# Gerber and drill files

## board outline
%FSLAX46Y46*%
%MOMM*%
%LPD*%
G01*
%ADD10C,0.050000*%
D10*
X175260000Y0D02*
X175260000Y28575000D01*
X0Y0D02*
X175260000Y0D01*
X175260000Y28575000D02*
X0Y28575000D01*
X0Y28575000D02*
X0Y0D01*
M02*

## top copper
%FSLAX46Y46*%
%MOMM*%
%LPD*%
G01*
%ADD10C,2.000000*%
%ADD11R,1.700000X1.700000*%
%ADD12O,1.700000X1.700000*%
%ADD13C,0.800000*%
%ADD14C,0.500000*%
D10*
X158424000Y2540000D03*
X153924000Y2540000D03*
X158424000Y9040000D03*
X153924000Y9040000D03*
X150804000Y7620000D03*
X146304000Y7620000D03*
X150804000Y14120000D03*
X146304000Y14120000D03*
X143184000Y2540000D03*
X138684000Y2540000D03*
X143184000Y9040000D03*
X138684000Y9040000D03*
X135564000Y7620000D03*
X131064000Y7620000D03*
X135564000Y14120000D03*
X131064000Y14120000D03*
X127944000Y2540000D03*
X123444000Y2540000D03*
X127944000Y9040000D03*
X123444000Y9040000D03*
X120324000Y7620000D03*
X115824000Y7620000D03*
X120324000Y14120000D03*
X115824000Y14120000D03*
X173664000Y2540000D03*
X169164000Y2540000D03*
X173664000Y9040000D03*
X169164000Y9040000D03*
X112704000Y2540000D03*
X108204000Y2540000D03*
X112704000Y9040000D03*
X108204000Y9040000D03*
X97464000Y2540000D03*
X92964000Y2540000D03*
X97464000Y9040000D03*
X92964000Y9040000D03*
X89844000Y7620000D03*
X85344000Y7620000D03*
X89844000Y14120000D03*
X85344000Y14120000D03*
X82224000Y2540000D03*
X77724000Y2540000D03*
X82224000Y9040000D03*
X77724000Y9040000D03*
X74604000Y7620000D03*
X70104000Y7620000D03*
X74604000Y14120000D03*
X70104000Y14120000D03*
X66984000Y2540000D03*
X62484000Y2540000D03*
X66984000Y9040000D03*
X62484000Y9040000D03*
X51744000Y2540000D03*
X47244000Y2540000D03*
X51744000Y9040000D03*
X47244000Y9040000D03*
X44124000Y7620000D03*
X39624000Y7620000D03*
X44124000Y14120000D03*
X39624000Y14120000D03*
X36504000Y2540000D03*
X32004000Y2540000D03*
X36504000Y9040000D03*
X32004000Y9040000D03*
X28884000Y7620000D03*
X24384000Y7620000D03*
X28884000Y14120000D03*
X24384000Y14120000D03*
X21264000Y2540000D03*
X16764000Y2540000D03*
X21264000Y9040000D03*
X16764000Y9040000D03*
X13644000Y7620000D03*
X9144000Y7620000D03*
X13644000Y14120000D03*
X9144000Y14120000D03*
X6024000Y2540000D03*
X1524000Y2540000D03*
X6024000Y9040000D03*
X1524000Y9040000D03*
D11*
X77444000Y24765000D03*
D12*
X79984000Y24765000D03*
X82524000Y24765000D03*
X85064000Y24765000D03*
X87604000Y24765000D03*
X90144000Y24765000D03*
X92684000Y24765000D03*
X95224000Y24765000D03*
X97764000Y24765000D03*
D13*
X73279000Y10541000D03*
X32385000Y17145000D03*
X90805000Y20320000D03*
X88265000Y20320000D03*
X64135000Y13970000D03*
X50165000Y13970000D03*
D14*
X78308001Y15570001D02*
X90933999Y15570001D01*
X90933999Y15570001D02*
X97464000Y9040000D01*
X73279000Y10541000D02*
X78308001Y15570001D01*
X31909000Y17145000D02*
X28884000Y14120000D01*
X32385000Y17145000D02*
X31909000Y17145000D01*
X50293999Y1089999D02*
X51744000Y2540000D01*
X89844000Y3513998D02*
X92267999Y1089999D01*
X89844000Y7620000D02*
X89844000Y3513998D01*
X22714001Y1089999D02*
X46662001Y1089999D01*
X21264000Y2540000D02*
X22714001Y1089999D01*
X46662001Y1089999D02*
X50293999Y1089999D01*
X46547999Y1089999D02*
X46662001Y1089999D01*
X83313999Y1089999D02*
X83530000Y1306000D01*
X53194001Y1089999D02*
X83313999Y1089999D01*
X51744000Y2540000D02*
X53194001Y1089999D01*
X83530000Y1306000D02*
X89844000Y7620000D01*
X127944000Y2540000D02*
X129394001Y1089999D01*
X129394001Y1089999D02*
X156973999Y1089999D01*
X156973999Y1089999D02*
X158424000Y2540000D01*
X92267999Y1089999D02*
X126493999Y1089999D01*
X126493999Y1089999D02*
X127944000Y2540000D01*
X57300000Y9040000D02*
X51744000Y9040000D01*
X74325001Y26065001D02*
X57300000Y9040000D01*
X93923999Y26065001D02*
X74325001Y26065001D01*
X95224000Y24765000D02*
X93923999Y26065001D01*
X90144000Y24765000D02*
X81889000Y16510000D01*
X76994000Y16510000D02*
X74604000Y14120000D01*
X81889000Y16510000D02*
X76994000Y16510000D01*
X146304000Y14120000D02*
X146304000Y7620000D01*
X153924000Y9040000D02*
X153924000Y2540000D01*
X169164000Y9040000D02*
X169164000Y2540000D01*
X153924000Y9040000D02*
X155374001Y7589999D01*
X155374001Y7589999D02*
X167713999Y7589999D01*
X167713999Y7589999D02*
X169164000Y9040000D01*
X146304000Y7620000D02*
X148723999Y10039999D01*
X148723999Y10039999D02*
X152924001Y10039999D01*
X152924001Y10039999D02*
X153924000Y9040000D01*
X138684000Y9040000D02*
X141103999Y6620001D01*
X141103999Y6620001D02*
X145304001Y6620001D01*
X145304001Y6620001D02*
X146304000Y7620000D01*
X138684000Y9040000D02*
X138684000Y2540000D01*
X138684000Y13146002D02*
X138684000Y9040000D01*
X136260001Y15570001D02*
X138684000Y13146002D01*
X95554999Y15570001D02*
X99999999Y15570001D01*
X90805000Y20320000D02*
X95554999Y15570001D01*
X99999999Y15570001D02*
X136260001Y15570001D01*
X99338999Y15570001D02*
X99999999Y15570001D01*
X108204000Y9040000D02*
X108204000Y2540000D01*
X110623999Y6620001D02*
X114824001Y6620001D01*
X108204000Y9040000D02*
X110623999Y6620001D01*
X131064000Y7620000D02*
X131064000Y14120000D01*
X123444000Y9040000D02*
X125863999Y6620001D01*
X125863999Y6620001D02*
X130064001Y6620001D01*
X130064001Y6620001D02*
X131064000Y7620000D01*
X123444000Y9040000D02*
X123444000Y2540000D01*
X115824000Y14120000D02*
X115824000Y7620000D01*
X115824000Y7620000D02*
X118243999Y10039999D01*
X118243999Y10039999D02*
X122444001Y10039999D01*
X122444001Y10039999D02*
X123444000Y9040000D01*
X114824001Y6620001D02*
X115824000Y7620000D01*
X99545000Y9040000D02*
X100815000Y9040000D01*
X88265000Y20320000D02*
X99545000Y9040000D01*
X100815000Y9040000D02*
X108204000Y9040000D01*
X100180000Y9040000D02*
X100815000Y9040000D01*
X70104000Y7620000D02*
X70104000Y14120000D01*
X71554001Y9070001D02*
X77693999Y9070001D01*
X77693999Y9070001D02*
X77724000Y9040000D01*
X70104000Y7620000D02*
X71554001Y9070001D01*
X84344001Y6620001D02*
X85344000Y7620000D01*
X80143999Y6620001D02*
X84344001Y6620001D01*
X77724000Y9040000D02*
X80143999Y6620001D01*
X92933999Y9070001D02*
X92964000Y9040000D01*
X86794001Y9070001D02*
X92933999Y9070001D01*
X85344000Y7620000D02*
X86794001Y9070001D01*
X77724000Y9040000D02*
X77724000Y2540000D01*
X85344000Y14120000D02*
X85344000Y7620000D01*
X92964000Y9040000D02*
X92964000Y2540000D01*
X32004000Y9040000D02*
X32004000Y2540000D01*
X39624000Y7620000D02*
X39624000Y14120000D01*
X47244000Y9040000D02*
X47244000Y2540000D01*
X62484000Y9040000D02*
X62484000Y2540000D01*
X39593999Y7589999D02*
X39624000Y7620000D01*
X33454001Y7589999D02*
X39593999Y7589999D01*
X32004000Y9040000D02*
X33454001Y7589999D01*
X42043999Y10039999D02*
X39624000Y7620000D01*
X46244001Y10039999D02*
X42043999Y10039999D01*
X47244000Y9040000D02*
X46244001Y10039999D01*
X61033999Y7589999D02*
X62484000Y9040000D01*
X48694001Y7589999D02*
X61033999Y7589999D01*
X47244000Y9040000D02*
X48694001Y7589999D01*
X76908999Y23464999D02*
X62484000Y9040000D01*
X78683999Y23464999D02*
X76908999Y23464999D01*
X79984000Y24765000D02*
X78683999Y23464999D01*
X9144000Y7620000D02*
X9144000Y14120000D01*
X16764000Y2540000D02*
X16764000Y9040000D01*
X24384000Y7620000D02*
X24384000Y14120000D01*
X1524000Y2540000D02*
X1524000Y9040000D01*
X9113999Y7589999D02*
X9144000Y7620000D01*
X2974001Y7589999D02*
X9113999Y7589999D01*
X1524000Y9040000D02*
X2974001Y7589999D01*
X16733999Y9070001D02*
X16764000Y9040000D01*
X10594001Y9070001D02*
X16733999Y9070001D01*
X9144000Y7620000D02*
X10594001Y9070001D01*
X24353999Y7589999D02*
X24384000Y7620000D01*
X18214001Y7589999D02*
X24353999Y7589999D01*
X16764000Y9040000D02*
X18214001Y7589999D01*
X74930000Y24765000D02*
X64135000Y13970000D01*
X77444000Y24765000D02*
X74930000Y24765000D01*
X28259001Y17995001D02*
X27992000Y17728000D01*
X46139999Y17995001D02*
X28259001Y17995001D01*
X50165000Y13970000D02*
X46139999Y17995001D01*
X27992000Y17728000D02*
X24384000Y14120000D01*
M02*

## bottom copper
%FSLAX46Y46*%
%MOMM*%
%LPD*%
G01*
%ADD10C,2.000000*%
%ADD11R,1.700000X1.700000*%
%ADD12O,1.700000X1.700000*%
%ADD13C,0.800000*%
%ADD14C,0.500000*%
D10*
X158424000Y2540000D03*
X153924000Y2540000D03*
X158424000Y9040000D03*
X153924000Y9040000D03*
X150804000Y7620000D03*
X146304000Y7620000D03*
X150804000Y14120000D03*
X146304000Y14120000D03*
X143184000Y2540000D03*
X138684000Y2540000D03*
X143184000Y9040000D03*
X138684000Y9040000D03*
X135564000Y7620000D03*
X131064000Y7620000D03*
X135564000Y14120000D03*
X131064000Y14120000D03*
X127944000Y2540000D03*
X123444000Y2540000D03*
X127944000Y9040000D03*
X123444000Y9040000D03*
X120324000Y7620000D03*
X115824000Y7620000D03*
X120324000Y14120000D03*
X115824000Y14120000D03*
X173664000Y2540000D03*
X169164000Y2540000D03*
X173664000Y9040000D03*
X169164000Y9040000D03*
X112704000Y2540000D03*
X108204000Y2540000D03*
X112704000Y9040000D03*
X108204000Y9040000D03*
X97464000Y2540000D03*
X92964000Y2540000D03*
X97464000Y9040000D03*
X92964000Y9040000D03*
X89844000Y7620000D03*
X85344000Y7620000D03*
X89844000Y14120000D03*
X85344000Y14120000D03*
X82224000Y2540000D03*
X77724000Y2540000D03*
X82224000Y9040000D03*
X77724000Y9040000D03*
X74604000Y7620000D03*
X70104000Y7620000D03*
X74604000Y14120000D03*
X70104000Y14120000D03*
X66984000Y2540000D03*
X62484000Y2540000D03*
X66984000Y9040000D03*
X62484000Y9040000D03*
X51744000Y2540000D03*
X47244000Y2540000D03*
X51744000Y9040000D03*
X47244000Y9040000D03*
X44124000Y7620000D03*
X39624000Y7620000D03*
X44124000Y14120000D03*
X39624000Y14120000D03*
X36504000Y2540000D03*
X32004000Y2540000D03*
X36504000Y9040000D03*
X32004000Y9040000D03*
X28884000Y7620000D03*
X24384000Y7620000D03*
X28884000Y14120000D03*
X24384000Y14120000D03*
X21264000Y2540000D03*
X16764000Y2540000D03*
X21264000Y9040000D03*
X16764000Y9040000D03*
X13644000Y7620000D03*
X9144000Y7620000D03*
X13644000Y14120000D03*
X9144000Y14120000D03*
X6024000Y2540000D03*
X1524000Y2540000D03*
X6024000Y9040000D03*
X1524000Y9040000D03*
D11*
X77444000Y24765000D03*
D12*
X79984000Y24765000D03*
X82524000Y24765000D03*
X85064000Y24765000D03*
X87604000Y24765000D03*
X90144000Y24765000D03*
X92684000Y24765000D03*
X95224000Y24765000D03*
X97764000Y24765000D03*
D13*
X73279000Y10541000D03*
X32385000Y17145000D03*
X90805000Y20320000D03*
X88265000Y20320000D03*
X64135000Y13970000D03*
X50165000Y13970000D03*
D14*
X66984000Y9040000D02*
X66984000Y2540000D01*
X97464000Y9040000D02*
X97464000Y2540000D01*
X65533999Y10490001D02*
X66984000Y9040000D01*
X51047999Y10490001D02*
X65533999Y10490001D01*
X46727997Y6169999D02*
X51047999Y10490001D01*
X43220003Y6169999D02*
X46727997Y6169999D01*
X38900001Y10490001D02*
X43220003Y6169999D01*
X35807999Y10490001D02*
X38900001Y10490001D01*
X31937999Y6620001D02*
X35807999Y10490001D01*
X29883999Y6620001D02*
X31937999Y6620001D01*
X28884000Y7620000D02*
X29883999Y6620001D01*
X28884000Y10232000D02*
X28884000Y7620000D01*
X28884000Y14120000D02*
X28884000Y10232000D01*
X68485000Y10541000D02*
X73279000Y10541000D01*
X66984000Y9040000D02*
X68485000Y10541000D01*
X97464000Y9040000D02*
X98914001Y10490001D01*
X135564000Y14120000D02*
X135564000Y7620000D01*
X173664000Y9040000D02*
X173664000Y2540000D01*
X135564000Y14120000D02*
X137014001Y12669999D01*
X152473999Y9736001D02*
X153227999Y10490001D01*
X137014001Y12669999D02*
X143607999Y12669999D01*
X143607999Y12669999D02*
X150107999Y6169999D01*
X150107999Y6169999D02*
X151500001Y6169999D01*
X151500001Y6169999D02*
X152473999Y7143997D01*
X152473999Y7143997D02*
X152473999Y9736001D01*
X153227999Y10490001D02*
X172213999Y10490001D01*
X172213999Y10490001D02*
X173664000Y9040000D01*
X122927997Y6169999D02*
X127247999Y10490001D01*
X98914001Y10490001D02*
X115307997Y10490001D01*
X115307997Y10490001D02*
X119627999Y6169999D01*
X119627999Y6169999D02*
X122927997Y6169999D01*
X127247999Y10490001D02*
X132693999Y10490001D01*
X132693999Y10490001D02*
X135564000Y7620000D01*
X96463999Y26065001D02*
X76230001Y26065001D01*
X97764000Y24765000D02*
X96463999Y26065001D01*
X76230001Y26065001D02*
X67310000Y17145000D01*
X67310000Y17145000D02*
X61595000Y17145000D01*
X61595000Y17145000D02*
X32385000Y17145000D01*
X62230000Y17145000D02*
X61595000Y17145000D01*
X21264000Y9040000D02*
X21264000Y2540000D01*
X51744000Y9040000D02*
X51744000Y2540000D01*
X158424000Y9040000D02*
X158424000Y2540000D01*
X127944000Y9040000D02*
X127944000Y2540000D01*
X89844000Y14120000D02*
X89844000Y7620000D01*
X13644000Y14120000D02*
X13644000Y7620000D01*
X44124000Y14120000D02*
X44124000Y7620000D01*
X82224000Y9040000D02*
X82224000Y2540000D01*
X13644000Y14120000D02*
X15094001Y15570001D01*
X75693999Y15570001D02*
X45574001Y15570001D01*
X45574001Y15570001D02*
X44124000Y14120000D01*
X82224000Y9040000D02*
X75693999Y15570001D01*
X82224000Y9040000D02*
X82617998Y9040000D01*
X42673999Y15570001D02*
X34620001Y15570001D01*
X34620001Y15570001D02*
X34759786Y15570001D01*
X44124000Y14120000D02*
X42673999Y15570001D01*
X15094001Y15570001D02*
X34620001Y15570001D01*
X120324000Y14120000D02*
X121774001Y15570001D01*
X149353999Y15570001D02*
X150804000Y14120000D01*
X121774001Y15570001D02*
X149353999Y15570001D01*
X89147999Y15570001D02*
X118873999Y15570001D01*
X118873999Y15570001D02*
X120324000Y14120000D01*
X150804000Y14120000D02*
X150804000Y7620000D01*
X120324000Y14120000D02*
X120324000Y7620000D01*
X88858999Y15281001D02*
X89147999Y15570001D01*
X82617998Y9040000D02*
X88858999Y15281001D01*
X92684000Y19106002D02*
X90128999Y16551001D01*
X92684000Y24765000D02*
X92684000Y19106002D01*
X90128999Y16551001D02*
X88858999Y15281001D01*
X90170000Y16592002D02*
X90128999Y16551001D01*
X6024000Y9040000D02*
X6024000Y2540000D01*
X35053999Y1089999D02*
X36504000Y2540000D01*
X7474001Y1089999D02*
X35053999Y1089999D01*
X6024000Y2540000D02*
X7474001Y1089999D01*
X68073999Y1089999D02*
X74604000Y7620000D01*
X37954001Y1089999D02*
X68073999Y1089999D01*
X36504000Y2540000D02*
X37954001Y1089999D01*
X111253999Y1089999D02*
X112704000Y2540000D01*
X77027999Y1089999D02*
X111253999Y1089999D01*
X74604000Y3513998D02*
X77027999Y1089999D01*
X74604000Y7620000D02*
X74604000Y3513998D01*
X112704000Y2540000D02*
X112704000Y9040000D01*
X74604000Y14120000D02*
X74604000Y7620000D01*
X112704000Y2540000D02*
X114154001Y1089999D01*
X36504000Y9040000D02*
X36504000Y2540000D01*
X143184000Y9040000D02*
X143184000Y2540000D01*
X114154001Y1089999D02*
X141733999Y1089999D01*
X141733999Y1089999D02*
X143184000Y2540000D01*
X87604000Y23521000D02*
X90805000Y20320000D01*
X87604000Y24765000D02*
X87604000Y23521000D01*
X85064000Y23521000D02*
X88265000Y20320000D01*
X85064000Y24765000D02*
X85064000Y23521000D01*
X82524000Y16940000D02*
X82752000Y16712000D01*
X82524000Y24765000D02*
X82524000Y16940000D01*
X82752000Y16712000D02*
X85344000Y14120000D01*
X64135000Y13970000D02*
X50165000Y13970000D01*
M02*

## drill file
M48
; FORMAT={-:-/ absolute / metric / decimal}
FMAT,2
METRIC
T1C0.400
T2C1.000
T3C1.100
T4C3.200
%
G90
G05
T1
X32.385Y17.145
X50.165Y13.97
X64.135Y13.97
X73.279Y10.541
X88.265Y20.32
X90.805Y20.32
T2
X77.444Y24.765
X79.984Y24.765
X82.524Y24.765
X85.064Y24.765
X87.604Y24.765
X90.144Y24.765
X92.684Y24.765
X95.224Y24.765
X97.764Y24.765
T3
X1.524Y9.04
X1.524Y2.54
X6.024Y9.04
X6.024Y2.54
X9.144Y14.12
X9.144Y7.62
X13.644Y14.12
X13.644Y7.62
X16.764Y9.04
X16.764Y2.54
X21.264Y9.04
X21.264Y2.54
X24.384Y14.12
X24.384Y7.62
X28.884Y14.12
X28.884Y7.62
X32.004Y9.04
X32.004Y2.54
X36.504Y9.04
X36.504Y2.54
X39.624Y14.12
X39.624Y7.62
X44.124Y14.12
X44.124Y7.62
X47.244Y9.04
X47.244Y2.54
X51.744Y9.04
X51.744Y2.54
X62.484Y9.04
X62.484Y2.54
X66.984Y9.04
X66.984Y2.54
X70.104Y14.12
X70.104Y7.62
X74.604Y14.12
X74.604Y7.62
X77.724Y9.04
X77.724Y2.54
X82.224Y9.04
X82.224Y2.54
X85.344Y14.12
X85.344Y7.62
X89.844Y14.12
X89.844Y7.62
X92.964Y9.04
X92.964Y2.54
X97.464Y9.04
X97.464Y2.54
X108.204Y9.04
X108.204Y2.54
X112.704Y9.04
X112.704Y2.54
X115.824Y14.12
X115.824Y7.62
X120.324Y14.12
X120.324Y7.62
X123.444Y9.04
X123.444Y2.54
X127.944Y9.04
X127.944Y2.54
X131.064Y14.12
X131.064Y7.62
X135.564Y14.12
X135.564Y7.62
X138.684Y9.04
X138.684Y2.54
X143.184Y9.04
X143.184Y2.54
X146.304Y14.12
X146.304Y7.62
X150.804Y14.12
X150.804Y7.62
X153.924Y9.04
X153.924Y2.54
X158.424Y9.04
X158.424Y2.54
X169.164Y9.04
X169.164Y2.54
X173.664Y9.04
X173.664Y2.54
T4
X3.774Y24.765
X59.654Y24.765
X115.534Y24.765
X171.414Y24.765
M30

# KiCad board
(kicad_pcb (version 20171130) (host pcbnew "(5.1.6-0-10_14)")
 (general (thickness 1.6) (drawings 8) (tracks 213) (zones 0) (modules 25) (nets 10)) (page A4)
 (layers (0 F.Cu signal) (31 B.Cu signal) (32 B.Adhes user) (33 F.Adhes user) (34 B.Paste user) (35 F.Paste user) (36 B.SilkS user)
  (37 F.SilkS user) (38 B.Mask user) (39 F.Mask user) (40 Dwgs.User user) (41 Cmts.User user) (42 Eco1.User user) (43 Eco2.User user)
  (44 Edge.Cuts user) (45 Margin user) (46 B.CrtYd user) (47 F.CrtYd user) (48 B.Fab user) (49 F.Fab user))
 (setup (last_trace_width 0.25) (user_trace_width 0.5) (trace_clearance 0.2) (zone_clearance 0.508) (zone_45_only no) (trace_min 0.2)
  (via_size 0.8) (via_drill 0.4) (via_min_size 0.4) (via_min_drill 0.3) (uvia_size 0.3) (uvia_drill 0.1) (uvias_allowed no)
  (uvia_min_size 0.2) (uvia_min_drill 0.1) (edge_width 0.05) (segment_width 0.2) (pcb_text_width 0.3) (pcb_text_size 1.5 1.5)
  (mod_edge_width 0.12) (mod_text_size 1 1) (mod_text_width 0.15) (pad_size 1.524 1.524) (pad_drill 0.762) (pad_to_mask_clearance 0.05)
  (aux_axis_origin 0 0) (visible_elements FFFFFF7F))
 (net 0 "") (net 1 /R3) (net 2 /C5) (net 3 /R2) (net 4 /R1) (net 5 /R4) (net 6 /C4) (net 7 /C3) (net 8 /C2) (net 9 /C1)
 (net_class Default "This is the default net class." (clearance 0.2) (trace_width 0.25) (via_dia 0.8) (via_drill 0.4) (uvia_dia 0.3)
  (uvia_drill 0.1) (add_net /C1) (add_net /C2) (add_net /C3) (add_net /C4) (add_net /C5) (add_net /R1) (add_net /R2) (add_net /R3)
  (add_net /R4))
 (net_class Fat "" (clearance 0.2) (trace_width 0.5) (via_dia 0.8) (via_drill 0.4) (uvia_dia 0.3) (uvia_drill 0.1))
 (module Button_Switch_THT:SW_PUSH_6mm (layer F.Cu) (at 153.924 -2.54 90)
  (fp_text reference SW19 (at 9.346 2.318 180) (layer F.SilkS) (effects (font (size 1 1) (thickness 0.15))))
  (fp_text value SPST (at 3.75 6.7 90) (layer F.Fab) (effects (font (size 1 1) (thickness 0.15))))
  (pad 2 thru_hole circle (at 0 4.5 180) (size 2 2) (drill 1.1) (layers *.Cu *.Mask) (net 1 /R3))
  (pad 1 thru_hole circle (at 0 0 180) (size 2 2) (drill 1.1) (layers *.Cu *.Mask) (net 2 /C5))
  (pad 2 thru_hole circle (at 6.5 4.5 180) (size 2 2) (drill 1.1) (layers *.Cu *.Mask) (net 1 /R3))
  (pad 1 thru_hole circle (at 6.5 0 180) (size 2 2) (drill 1.1) (layers *.Cu *.Mask) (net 2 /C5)))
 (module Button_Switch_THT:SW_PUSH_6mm (layer F.Cu) (at 146.304 -7.62 90)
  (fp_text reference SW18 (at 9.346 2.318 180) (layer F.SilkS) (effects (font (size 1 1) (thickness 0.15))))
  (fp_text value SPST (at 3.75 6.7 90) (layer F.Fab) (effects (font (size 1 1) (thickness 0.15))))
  (pad 2 thru_hole circle (at 0 4.5 180) (size 2 2) (drill 1.1) (layers *.Cu *.Mask) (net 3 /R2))
  (pad 1 thru_hole circle (at 0 0 180) (size 2 2) (drill 1.1) (layers *.Cu *.Mask) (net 2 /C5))
  (pad 2 thru_hole circle (at 6.5 4.5 180) (size 2 2) (drill 1.1) (layers *.Cu *.Mask) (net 3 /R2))
  (pad 1 thru_hole circle (at 6.5 0 180) (size 2 2) (drill 1.1) (layers *.Cu *.Mask) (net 2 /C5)))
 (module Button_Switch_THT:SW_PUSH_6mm (layer F.Cu) (at 138.684 -2.54 90)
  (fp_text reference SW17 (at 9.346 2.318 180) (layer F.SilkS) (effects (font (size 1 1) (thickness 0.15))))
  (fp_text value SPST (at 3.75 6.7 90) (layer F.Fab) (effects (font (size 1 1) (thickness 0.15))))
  (pad 2 thru_hole circle (at 0 4.5 180) (size 2 2) (drill 1.1) (layers *.Cu *.Mask) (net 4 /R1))
  (pad 1 thru_hole circle (at 0 0 180) (size 2 2) (drill 1.1) (layers *.Cu *.Mask) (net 2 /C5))
  (pad 2 thru_hole circle (at 6.5 4.5 180) (size 2 2) (drill 1.1) (layers *.Cu *.Mask) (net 4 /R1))
  (pad 1 thru_hole circle (at 6.5 0 180) (size 2 2) (drill 1.1) (layers *.Cu *.Mask) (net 2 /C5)))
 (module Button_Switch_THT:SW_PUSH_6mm (layer F.Cu) (at 131.064 -7.62 90)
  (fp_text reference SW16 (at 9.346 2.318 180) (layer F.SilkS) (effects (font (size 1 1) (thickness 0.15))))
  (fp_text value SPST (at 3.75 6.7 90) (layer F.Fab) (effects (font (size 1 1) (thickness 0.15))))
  (pad 2 thru_hole circle (at 0 4.5 180) (size 2 2) (drill 1.1) (layers *.Cu *.Mask) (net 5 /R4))
  (pad 1 thru_hole circle (at 0 0 180) (size 2 2) (drill 1.1) (layers *.Cu *.Mask) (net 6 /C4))
  (pad 2 thru_hole circle (at 6.5 4.5 180) (size 2 2) (drill 1.1) (layers *.Cu *.Mask) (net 5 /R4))
  (pad 1 thru_hole circle (at 6.5 0 180) (size 2 2) (drill 1.1) (layers *.Cu *.Mask) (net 6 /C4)))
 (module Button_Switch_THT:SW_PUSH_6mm (layer F.Cu) (at 123.444 -2.54 90)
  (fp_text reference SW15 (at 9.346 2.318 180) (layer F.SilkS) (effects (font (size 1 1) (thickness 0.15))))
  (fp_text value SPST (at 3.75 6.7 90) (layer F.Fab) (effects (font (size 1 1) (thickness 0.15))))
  (pad 2 thru_hole circle (at 0 4.5 180) (size 2 2) (drill 1.1) (layers *.Cu *.Mask) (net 1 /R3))
  (pad 1 thru_hole circle (at 0 0 180) (size 2 2) (drill 1.1) (layers *.Cu *.Mask) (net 6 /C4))
  (pad 2 thru_hole circle (at 6.5 4.5 180) (size 2 2) (drill 1.1) (layers *.Cu *.Mask) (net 1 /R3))
  (pad 1 thru_hole circle (at 6.5 0 180) (size 2 2) (drill 1.1) (layers *.Cu *.Mask) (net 6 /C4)))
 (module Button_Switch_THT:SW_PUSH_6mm (layer F.Cu) (at 115.824 -7.62 90)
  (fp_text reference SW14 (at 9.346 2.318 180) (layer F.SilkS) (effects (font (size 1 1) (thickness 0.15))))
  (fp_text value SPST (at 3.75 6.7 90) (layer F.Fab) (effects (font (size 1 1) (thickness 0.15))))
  (pad 2 thru_hole circle (at 0 4.5 180) (size 2 2) (drill 1.1) (layers *.Cu *.Mask) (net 3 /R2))
  (pad 1 thru_hole circle (at 0 0 180) (size 2 2) (drill 1.1) (layers *.Cu *.Mask) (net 6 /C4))
  (pad 2 thru_hole circle (at 6.5 4.5 180) (size 2 2) (drill 1.1) (layers *.Cu *.Mask) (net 3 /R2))
  (pad 1 thru_hole circle (at 6.5 0 180) (size 2 2) (drill 1.1) (layers *.Cu *.Mask) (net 6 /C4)))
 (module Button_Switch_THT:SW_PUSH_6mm (layer F.Cu) (at 169.164 -2.54 90)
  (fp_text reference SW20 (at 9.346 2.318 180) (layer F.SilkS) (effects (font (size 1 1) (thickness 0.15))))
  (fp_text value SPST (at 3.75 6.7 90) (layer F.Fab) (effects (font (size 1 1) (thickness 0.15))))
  (pad 2 thru_hole circle (at 0 4.5 180) (size 2 2) (drill 1.1) (layers *.Cu *.Mask) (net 5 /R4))
  (pad 1 thru_hole circle (at 0 0 180) (size 2 2) (drill 1.1) (layers *.Cu *.Mask) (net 2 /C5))
  (pad 2 thru_hole circle (at 6.5 4.5 180) (size 2 2) (drill 1.1) (layers *.Cu *.Mask) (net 5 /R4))
  (pad 1 thru_hole circle (at 6.5 0 180) (size 2 2) (drill 1.1) (layers *.Cu *.Mask) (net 2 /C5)))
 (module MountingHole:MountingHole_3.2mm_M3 (layer F.Cu) (at 115.534 -24.765)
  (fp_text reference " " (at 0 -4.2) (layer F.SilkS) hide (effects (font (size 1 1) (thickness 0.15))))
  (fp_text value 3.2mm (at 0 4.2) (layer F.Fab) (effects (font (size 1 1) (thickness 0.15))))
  (pad 1 np_thru_hole circle (at 0 0) (size 3.2 3.2) (drill 3.2) (layers *.Cu *.Mask)))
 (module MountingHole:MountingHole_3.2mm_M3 (layer F.Cu) (at 59.654 -24.765)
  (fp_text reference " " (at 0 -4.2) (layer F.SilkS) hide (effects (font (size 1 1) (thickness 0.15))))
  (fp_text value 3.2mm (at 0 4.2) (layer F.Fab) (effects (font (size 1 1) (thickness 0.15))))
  (pad 1 np_thru_hole circle (at 0 0) (size 3.2 3.2) (drill 3.2) (layers *.Cu *.Mask)))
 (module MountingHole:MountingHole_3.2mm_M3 (layer F.Cu) (at 171.414 -24.765)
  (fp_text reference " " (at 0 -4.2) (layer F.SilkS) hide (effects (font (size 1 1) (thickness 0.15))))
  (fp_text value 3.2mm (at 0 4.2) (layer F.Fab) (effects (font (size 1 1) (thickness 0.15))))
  (pad 1 np_thru_hole circle (at 0 0) (size 3.2 3.2) (drill 3.2) (layers *.Cu *.Mask)))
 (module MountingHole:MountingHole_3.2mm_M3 (layer F.Cu) (at 3.774 -24.765)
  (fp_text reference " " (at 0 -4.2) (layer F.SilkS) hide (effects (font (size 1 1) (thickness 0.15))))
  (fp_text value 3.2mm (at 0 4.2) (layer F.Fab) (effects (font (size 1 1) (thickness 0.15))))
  (pad 1 np_thru_hole circle (at 0 0) (size 3.2 3.2) (drill 3.2) (layers *.Cu *.Mask)))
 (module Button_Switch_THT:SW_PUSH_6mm (layer F.Cu) (at 108.204 -2.54 90)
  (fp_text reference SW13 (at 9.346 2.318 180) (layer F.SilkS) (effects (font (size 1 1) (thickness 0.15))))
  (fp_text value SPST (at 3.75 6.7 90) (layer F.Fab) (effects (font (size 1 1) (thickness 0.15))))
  (pad 2 thru_hole circle (at 0 4.5 180) (size 2 2) (drill 1.1) (layers *.Cu *.Mask) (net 4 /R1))
  (pad 1 thru_hole circle (at 0 0 180) (size 2 2) (drill 1.1) (layers *.Cu *.Mask) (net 6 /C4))
  (pad 2 thru_hole circle (at 6.5 4.5 180) (size 2 2) (drill 1.1) (layers *.Cu *.Mask) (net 4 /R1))
  (pad 1 thru_hole circle (at 6.5 0 180) (size 2 2) (drill 1.1) (layers *.Cu *.Mask) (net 6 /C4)))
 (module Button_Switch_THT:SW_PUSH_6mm (layer F.Cu) (at 92.964 -2.54 90)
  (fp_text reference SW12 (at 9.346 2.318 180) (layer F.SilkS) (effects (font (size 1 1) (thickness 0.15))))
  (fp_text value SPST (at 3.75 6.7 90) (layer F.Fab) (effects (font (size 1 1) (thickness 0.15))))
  (pad 2 thru_hole circle (at 0 4.5 180) (size 2 2) (drill 1.1) (layers *.Cu *.Mask) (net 5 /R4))
  (pad 1 thru_hole circle (at 0 0 180) (size 2 2) (drill 1.1) (layers *.Cu *.Mask) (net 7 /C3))
  (pad 2 thru_hole circle (at 6.5 4.5 180) (size 2 2) (drill 1.1) (layers *.Cu *.Mask) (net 5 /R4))
  (pad 1 thru_hole circle (at 6.5 0 180) (size 2 2) (drill 1.1) (layers *.Cu *.Mask) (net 7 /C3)))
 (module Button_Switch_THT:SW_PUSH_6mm (layer F.Cu) (at 85.344 -7.62 90)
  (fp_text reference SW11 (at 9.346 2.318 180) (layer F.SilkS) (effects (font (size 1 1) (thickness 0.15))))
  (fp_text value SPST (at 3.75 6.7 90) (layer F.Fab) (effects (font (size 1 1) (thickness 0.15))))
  (pad 2 thru_hole circle (at 0 4.5 180) (size 2 2) (drill 1.1) (layers *.Cu *.Mask) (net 1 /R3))
  (pad 1 thru_hole circle (at 0 0 180) (size 2 2) (drill 1.1) (layers *.Cu *.Mask) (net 7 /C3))
  (pad 2 thru_hole circle (at 6.5 4.5 180) (size 2 2) (drill 1.1) (layers *.Cu *.Mask) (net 1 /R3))
  (pad 1 thru_hole circle (at 6.5 0 180) (size 2 2) (drill 1.1) (layers *.Cu *.Mask) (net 7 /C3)))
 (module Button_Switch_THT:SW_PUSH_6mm (layer F.Cu) (at 77.724 -2.54 90)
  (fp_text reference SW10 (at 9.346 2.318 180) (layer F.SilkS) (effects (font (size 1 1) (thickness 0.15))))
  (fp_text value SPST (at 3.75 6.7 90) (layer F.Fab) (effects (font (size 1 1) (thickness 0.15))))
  (pad 2 thru_hole circle (at 0 4.5 180) (size 2 2) (drill 1.1) (layers *.Cu *.Mask) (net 3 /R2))
  (pad 1 thru_hole circle (at 0 0 180) (size 2 2) (drill 1.1) (layers *.Cu *.Mask) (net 7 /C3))
  (pad 2 thru_hole circle (at 6.5 4.5 180) (size 2 2) (drill 1.1) (layers *.Cu *.Mask) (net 3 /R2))
  (pad 1 thru_hole circle (at 6.5 0 180) (size 2 2) (drill 1.1) (layers *.Cu *.Mask) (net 7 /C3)))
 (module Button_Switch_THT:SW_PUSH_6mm (layer F.Cu) (at 70.104 -7.62 90)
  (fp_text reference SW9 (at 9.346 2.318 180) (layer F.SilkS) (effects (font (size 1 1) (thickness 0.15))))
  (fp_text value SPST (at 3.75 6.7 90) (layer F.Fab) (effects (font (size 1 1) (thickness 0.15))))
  (pad 2 thru_hole circle (at 0 4.5 180) (size 2 2) (drill 1.1) (layers *.Cu *.Mask) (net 4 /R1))
  (pad 1 thru_hole circle (at 0 0 180) (size 2 2) (drill 1.1) (layers *.Cu *.Mask) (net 7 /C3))
  (pad 2 thru_hole circle (at 6.5 4.5 180) (size 2 2) (drill 1.1) (layers *.Cu *.Mask) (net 4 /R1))
  (pad 1 thru_hole circle (at 6.5 0 180) (size 2 2) (drill 1.1) (layers *.Cu *.Mask) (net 7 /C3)))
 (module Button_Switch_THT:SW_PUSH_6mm (layer F.Cu) (at 62.484 -2.54 90)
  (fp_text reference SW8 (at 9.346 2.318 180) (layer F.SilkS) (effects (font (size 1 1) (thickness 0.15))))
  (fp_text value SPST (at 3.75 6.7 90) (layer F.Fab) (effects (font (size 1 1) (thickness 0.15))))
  (pad 2 thru_hole circle (at 0 4.5 180) (size 2 2) (drill 1.1) (layers *.Cu *.Mask) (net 5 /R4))
  (pad 1 thru_hole circle (at 0 0 180) (size 2 2) (drill 1.1) (layers *.Cu *.Mask) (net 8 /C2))
  (pad 2 thru_hole circle (at 6.5 4.5 180) (size 2 2) (drill 1.1) (layers *.Cu *.Mask) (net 5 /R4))
  (pad 1 thru_hole circle (at 6.5 0 180) (size 2 2) (drill 1.1) (layers *.Cu *.Mask) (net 8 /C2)))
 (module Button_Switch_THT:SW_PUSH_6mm (layer F.Cu) (at 47.244 -2.54 90)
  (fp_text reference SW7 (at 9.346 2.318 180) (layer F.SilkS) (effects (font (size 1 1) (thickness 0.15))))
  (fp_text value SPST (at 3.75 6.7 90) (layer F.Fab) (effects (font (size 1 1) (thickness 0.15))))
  (pad 2 thru_hole circle (at 0 4.5 180) (size 2 2) (drill 1.1) (layers *.Cu *.Mask) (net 1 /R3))
  (pad 1 thru_hole circle (at 0 0 180) (size 2 2) (drill 1.1) (layers *.Cu *.Mask) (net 8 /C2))
  (pad 2 thru_hole circle (at 6.5 4.5 180) (size 2 2) (drill 1.1) (layers *.Cu *.Mask) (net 1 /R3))
  (pad 1 thru_hole circle (at 6.5 0 180) (size 2 2) (drill 1.1) (layers *.Cu *.Mask) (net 8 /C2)))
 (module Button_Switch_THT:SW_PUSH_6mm (layer F.Cu) (at 39.624 -7.62 90)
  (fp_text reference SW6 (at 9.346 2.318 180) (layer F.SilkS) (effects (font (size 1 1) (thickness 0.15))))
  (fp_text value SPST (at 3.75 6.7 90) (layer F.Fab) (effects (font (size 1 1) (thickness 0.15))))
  (pad 2 thru_hole circle (at 0 4.5 180) (size 2 2) (drill 1.1) (layers *.Cu *.Mask) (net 3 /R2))
  (pad 1 thru_hole circle (at 0 0 180) (size 2 2) (drill 1.1) (layers *.Cu *.Mask) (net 8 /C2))
  (pad 2 thru_hole circle (at 6.5 4.5 180) (size 2 2) (drill 1.1) (layers *.Cu *.Mask) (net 3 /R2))
  (pad 1 thru_hole circle (at 6.5 0 180) (size 2 2) (drill 1.1) (layers *.Cu *.Mask) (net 8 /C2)))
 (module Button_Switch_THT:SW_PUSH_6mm (layer F.Cu) (at 32.004 -2.54 90)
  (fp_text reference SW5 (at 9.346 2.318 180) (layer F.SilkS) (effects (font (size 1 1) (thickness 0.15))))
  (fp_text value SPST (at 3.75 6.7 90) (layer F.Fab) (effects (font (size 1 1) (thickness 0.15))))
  (pad 2 thru_hole circle (at 0 4.5 180) (size 2 2) (drill 1.1) (layers *.Cu *.Mask) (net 4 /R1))
  (pad 1 thru_hole circle (at 0 0 180) (size 2 2) (drill 1.1) (layers *.Cu *.Mask) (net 8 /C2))
  (pad 2 thru_hole circle (at 6.5 4.5 180) (size 2 2) (drill 1.1) (layers *.Cu *.Mask) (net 4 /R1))
  (pad 1 thru_hole circle (at 6.5 0 180) (size 2 2) (drill 1.1) (layers *.Cu *.Mask) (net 8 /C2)))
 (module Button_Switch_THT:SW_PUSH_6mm (layer F.Cu) (at 24.384 -7.62 90)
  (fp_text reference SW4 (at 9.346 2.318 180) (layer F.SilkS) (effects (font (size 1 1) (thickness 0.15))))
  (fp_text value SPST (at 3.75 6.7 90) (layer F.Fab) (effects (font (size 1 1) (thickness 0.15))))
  (pad 2 thru_hole circle (at 0 4.5 180) (size 2 2) (drill 1.1) (layers *.Cu *.Mask) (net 5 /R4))
  (pad 1 thru_hole circle (at 0 0 180) (size 2 2) (drill 1.1) (layers *.Cu *.Mask) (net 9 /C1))
  (pad 2 thru_hole circle (at 6.5 4.5 180) (size 2 2) (drill 1.1) (layers *.Cu *.Mask) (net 5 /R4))
  (pad 1 thru_hole circle (at 6.5 0 180) (size 2 2) (drill 1.1) (layers *.Cu *.Mask) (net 9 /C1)))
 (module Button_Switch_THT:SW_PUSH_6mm (layer F.Cu) (at 16.764 -2.54 90)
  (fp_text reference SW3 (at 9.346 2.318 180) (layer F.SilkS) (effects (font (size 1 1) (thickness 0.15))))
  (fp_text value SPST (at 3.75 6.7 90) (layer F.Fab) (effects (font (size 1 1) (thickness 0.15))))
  (pad 2 thru_hole circle (at 0 4.5 180) (size 2 2) (drill 1.1) (layers *.Cu *.Mask) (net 1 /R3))
  (pad 1 thru_hole circle (at 0 0 180) (size 2 2) (drill 1.1) (layers *.Cu *.Mask) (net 9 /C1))
  (pad 2 thru_hole circle (at 6.5 4.5 180) (size 2 2) (drill 1.1) (layers *.Cu *.Mask) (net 1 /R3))
  (pad 1 thru_hole circle (at 6.5 0 180) (size 2 2) (drill 1.1) (layers *.Cu *.Mask) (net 9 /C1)))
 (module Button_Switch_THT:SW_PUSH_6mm (layer F.Cu) (at 9.144 -7.62 90)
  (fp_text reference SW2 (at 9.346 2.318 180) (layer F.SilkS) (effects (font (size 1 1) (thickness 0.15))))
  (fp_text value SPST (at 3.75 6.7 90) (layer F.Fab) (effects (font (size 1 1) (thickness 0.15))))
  (pad 2 thru_hole circle (at 0 4.5 180) (size 2 2) (drill 1.1) (layers *.Cu *.Mask) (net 3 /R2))
  (pad 1 thru_hole circle (at 0 0 180) (size 2 2) (drill 1.1) (layers *.Cu *.Mask) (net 9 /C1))
  (pad 2 thru_hole circle (at 6.5 4.5 180) (size 2 2) (drill 1.1) (layers *.Cu *.Mask) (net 3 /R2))
  (pad 1 thru_hole circle (at 6.5 0 180) (size 2 2) (drill 1.1) (layers *.Cu *.Mask) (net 9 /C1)))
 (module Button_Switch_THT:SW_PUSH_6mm (layer F.Cu) (at 1.524 -2.54 90)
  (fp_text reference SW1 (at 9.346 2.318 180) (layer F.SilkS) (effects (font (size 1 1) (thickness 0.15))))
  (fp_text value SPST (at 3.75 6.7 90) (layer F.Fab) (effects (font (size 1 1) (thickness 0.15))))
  (pad 2 thru_hole circle (at 0 4.5 180) (size 2 2) (drill 1.1) (layers *.Cu *.Mask) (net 4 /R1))
  (pad 1 thru_hole circle (at 0 0 180) (size 2 2) (drill 1.1) (layers *.Cu *.Mask) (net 9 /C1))
  (pad 2 thru_hole circle (at 6.5 4.5 180) (size 2 2) (drill 1.1) (layers *.Cu *.Mask) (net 4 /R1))
  (pad 1 thru_hole circle (at 6.5 0 180) (size 2 2) (drill 1.1) (layers *.Cu *.Mask) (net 9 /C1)))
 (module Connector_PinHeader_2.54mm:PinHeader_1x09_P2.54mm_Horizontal (layer F.Cu) (at 77.444 -24.765 90)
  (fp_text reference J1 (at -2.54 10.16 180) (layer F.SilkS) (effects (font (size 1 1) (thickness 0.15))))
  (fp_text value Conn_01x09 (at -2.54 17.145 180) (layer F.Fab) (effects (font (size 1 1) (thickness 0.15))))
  (pad 1 thru_hole rect (at 0 0 90) (size 1.7 1.7) (drill 1) (layers *.Cu *.Mask) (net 9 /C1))
  (pad 2 thru_hole oval (at 0 2.54 90) (size 1.7 1.7) (drill 1) (layers *.Cu *.Mask) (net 8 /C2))
  (pad 3 thru_hole oval (at 0 5.08 90) (size 1.7 1.7) (drill 1) (layers *.Cu *.Mask) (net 7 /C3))
  (pad 4 thru_hole oval (at 0 7.62 90) (size 1.7 1.7) (drill 1) (layers *.Cu *.Mask) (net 6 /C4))
  (pad 5 thru_hole oval (at 0 10.16 90) (size 1.7 1.7) (drill 1) (layers *.Cu *.Mask) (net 2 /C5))
  (pad 6 thru_hole oval (at 0 12.7 90) (size 1.7 1.7) (drill 1) (layers *.Cu *.Mask) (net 4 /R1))
  (pad 7 thru_hole oval (at 0 15.24 90) (size 1.7 1.7) (drill 1) (layers *.Cu *.Mask) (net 3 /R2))
  (pad 8 thru_hole oval (at 0 17.78 90) (size 1.7 1.7) (drill 1) (layers *.Cu *.Mask) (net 1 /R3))
  (pad 9 thru_hole oval (at 0 20.32 90) (size 1.7 1.7) (drill 1) (layers *.Cu *.Mask) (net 5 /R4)))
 (gr_line (start 175.26 0) (end 175.26 -28.575) (layer Edge.Cuts) (width 0.05))
 (gr_line (start 0 0) (end 175.26 0) (layer Edge.Cuts) (width 0.05))
 (gr_line (start 175.26 -28.575) (end 0 -28.575) (layer Edge.Cuts) (width 0.05))
 (gr_line (start 0 -28.575) (end 0 0) (layer Edge.Cuts) (width 0.05))
 (segment (start 66.984 -9.04) (end 66.984 -2.54) (width 0.5) (layer B.Cu) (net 5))
 (segment (start 97.464 -9.04) (end 97.464 -2.54) (width 0.5) (layer B.Cu) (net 5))
 (segment (start 65.533999 -10.490001) (end 66.984 -9.04) (width 0.5) (layer B.Cu) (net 5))
 (segment (start 51.047999 -10.490001) (end 65.533999 -10.490001) (width 0.5) (layer B.Cu) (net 5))
 (segment (start 46.727997 -6.169999) (end 51.047999 -10.490001) (width 0.5) (layer B.Cu) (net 5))
 (segment (start 43.220003 -6.169999) (end 46.727997 -6.169999) (width 0.5) (layer B.Cu) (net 5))
 (segment (start 38.900001 -10.490001) (end 43.220003 -6.169999) (width 0.5) (layer B.Cu) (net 5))
 (segment (start 35.807999 -10.490001) (end 38.900001 -10.490001) (width 0.5) (layer B.Cu) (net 5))
 (segment (start 31.937999 -6.620001) (end 35.807999 -10.490001) (width 0.5) (layer B.Cu) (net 5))
 (segment (start 29.883999 -6.620001) (end 31.937999 -6.620001) (width 0.5) (layer B.Cu) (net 5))
 (segment (start 28.884 -7.62) (end 29.883999 -6.620001) (width 0.5) (layer B.Cu) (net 5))
 (segment (start 28.884 -10.232) (end 28.884 -7.62) (width 0.5) (layer B.Cu) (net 5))
 (segment (start 28.884 -14.12) (end 28.884 -10.232) (width 0.5) (layer B.Cu) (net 5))
 (segment (start 68.485 -10.541) (end 73.279 -10.541) (width 0.5) (layer B.Cu) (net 5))
 (via (at 73.279 -10.541) (size 0.8) (drill 0.4) (layers F.Cu B.Cu) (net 5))
 (segment (start 66.984 -9.04) (end 68.485 -10.541) (width 0.5) (layer B.Cu) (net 5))
 (segment (start 78.308001 -15.570001) (end 90.933999 -15.570001) (width 0.5) (layer F.Cu) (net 5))
 (segment (start 90.933999 -15.570001) (end 97.464 -9.04) (width 0.5) (layer F.Cu) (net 5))
 (segment (start 73.279 -10.541) (end 78.308001 -15.570001) (width 0.5) (layer F.Cu) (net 5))
 (segment (start 97.464 -9.04) (end 98.914001 -10.490001) (width 0.5) (layer B.Cu) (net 5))
 (segment (start 135.564 -14.12) (end 135.564 -7.62) (width 0.5) (layer B.Cu) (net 5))
 (segment (start 173.664 -9.04) (end 173.664 -2.54) (width 0.5) (layer B.Cu) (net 5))
 (segment (start 135.564 -14.12) (end 137.014001 -12.669999) (width 0.5) (layer B.Cu) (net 5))
 (segment (start 152.473999 -9.736001) (end 153.227999 -10.490001) (width 0.5) (layer B.Cu) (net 5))
 (segment (start 137.014001 -12.669999) (end 143.607999 -12.669999) (width 0.5) (layer B.Cu) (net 5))
 (segment (start 143.607999 -12.669999) (end 150.107999 -6.169999) (width 0.5) (layer B.Cu) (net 5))
 (segment (start 150.107999 -6.169999) (end 151.500001 -6.169999) (width 0.5) (layer B.Cu) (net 5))
 (segment (start 151.500001 -6.169999) (end 152.473999 -7.143997) (width 0.5) (layer B.Cu) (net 5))
 (segment (start 152.473999 -7.143997) (end 152.473999 -9.736001) (width 0.5) (layer B.Cu) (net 5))
 (segment (start 153.227999 -10.490001) (end 172.213999 -10.490001) (width 0.5) (layer B.Cu) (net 5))
 (segment (start 172.213999 -10.490001) (end 173.664 -9.04) (width 0.5) (layer B.Cu) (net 5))
 (segment (start 122.927997 -6.169999) (end 127.247999 -10.490001) (width 0.5) (layer B.Cu) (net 5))
 (segment (start 98.914001 -10.490001) (end 115.307997 -10.490001) (width 0.5) (layer B.Cu) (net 5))
 (segment (start 115.307997 -10.490001) (end 119.627999 -6.169999) (width 0.5) (layer B.Cu) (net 5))
 (segment (start 119.627999 -6.169999) (end 122.927997 -6.169999) (width 0.5) (layer B.Cu) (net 5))
 (segment (start 127.247999 -10.490001) (end 132.693999 -10.490001) (width 0.5) (layer B.Cu) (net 5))
 (segment (start 132.693999 -10.490001) (end 135.564 -7.62) (width 0.5) (layer B.Cu) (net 5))
 (via (at 32.385 -17.145) (size 0.8) (drill 0.4) (layers F.Cu B.Cu) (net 5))
 (segment (start 31.909 -17.145) (end 28.884 -14.12) (width 0.5) (layer F.Cu) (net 5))
 (segment (start 32.385 -17.145) (end 31.909 -17.145) (width 0.5) (layer F.Cu) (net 5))
 (segment (start 96.463999 -26.065001) (end 76.230001 -26.065001) (width 0.5) (layer B.Cu) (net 5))
 (segment (start 97.764 -24.765) (end 96.463999 -26.065001) (width 0.5) (layer B.Cu) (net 5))
 (segment (start 76.230001 -26.065001) (end 67.31 -17.145) (width 0.5) (layer B.Cu) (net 5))
 (segment (start 67.31 -17.145) (end 61.595 -17.145) (width 0.5) (layer B.Cu) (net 5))
 (segment (start 61.595 -17.145) (end 32.385 -17.145) (width 0.5) (layer B.Cu) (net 5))
 (segment (start 62.23 -17.145) (end 61.595 -17.145) (width 0.5) (layer B.Cu) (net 5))
 (segment (start 21.264 -9.04) (end 21.264 -2.54) (width 0.5) (layer B.Cu) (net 1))
 (segment (start 51.744 -9.04) (end 51.744 -2.54) (width 0.5) (layer B.Cu) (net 1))
 (segment (start 50.293999 -1.089999) (end 51.744 -2.54) (width 0.5) (layer F.Cu) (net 1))
 (segment (start 89.844 -3.513998) (end 92.267999 -1.089999) (width 0.5) (layer F.Cu) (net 1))
 (segment (start 89.844 -7.62) (end 89.844 -3.513998) (width 0.5) (layer F.Cu) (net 1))
 (segment (start 22.714001 -1.089999) (end 46.662001 -1.089999) (width 0.5) (layer F.Cu) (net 1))
 (segment (start 21.264 -2.54) (end 22.714001 -1.089999) (width 0.5) (layer F.Cu) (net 1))
 (segment (start 46.662001 -1.089999) (end 50.293999 -1.089999) (width 0.5) (layer F.Cu) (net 1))
 (segment (start 46.547999 -1.089999) (end 46.662001 -1.089999) (width 0.5) (layer F.Cu) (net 1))
 (segment (start 83.313999 -1.089999) (end 83.53 -1.306) (width 0.5) (layer F.Cu) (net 1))
 (segment (start 53.194001 -1.089999) (end 83.313999 -1.089999) (width 0.5) (layer F.Cu) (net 1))
 (segment (start 51.744 -2.54) (end 53.194001 -1.089999) (width 0.5) (layer F.Cu) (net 1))
 (segment (start 83.53 -1.306) (end 89.844 -7.62) (width 0.5) (layer F.Cu) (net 1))
 (segment (start 127.944 -2.54) (end 129.394001 -1.089999) (width 0.5) (layer F.Cu) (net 1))
 (segment (start 129.394001 -1.089999) (end 156.973999 -1.089999) (width 0.5) (layer F.Cu) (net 1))
 (segment (start 156.973999 -1.089999) (end 158.424 -2.54) (width 0.5) (layer F.Cu) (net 1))
 (segment (start 92.267999 -1.089999) (end 126.493999 -1.089999) (width 0.5) (layer F.Cu) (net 1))
 (segment (start 126.493999 -1.089999) (end 127.944 -2.54) (width 0.5) (layer F.Cu) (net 1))
 (segment (start 158.424 -9.04) (end 158.424 -2.54) (width 0.5) (layer B.Cu) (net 1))
 (segment (start 127.944 -9.04) (end 127.944 -2.54) (width 0.5) (layer B.Cu) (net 1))
 (segment (start 89.844 -14.12) (end 89.844 -7.62) (width 0.5) (layer B.Cu) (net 1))
 (segment (start 57.3 -9.04) (end 51.744 -9.04) (width 0.5) (layer F.Cu) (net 1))
 (segment (start 74.325001 -26.065001) (end 57.3 -9.04) (width 0.5) (layer F.Cu) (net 1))
 (segment (start 93.923999 -26.065001) (end 74.325001 -26.065001) (width 0.5) (layer F.Cu) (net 1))
 (segment (start 95.224 -24.765) (end 93.923999 -26.065001) (width 0.5) (layer F.Cu) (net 1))
 (segment (start 13.644 -14.12) (end 13.644 -7.62) (width 0.5) (layer B.Cu) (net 3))
 (segment (start 44.124 -14.12) (end 44.124 -7.62) (width 0.5) (layer B.Cu) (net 3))
 (segment (start 82.224 -9.04) (end 82.224 -2.54) (width 0.5) (layer B.Cu) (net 3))
 (segment (start 13.644 -14.12) (end 15.094001 -15.570001) (width 0.5) (layer B.Cu) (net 3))
 (segment (start 75.693999 -15.570001) (end 45.574001 -15.570001) (width 0.5) (layer B.Cu) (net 3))
 (segment (start 45.574001 -15.570001) (end 44.124 -14.12) (width 0.5) (layer B.Cu) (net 3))
 (segment (start 82.224 -9.04) (end 75.693999 -15.570001) (width 0.5) (layer B.Cu) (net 3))
 (segment (start 82.224 -9.04) (end 82.617998 -9.04) (width 0.5) (layer B.Cu) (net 3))
 (segment (start 42.673999 -15.570001) (end 34.620001 -15.570001) (width 0.5) (layer B.Cu) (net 3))
 (segment (start 34.620001 -15.570001) (end 34.759786 -15.570001) (width 0.5) (layer B.Cu) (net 3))
 (segment (start 44.124 -14.12) (end 42.673999 -15.570001) (width 0.5) (layer B.Cu) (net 3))
 (segment (start 15.094001 -15.570001) (end 34.620001 -15.570001) (width 0.5) (layer B.Cu) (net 3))
 (segment (start 120.324 -14.12) (end 121.774001 -15.570001) (width 0.5) (layer B.Cu) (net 3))
 (segment (start 149.353999 -15.570001) (end 150.804 -14.12) (width 0.5) (layer B.Cu) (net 3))
 (segment (start 121.774001 -15.570001) (end 149.353999 -15.570001) (width 0.5) (layer B.Cu) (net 3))
 (segment (start 89.147999 -15.570001) (end 118.873999 -15.570001) (width 0.5) (layer B.Cu) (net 3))
 (segment (start 118.873999 -15.570001) (end 120.324 -14.12) (width 0.5) (layer B.Cu) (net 3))
 (segment (start 150.804 -14.12) (end 150.804 -7.62) (width 0.5) (layer B.Cu) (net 3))
 (segment (start 120.324 -14.12) (end 120.324 -7.62) (width 0.5) (layer B.Cu) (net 3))
 (segment (start 88.858999 -15.281001) (end 89.147999 -15.570001) (width 0.5) (layer B.Cu) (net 3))
 (segment (start 82.617998 -9.04) (end 88.858999 -15.281001) (width 0.5) (layer B.Cu) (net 3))
 (segment (start 92.684 -19.106002) (end 90.128999 -16.551001) (width 0.5) (layer B.Cu) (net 3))
 (segment (start 92.684 -24.765) (end 92.684 -19.106002) (width 0.5) (layer B.Cu) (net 3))
 (segment (start 90.128999 -16.551001) (end 88.858999 -15.281001) (width 0.5) (layer B.Cu) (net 3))
 (segment (start 90.17 -16.592002) (end 90.128999 -16.551001) (width 0.5) (layer B.Cu) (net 3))
 (segment (start 6.024 -9.04) (end 6.024 -2.54) (width 0.5) (layer B.Cu) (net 4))
 (segment (start 35.053999 -1.089999) (end 36.504 -2.54) (width 0.5) (layer B.Cu) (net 4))
 (segment (start 7.474001 -1.089999) (end 35.053999 -1.089999) (width 0.5) (layer B.Cu) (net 4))
 (segment (start 6.024 -2.54) (end 7.474001 -1.089999) (width 0.5) (layer B.Cu) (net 4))
 (segment (start 68.073999 -1.089999) (end 74.604 -7.62) (width 0.5) (layer B.Cu) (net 4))
 (segment (start 37.954001 -1.089999) (end 68.073999 -1.089999) (width 0.5) (layer B.Cu) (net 4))
 (segment (start 36.504 -2.54) (end 37.954001 -1.089999) (width 0.5) (layer B.Cu) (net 4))
 (segment (start 111.253999 -1.089999) (end 112.704 -2.54) (width 0.5) (layer B.Cu) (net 4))
 (segment (start 77.027999 -1.089999) (end 111.253999 -1.089999) (width 0.5) (layer B.Cu) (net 4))
 (segment (start 74.604 -3.513998) (end 77.027999 -1.089999) (width 0.5) (layer B.Cu) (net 4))
 (segment (start 74.604 -7.62) (end 74.604 -3.513998) (width 0.5) (layer B.Cu) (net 4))
 (segment (start 112.704 -2.54) (end 112.704 -9.04) (width 0.5) (layer B.Cu) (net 4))
 (segment (start 74.604 -14.12) (end 74.604 -7.62) (width 0.5) (layer B.Cu) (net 4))
 (segment (start 112.704 -2.54) (end 114.154001 -1.089999) (width 0.5) (layer B.Cu) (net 4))
 (segment (start 36.504 -9.04) (end 36.504 -2.54) (width 0.5) (layer B.Cu) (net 4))
 (segment (start 143.184 -9.04) (end 143.184 -2.54) (width 0.5) (layer B.Cu) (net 4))
 (segment (start 114.154001 -1.089999) (end 141.733999 -1.089999) (width 0.5) (layer B.Cu) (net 4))
 (segment (start 141.733999 -1.089999) (end 143.184 -2.54) (width 0.5) (layer B.Cu) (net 4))
 (segment (start 90.144 -24.765) (end 81.889 -16.51) (width 0.5) (layer F.Cu) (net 4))
 (segment (start 76.994 -16.51) (end 74.604 -14.12) (width 0.5) (layer F.Cu) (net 4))
 (segment (start 81.889 -16.51) (end 76.994 -16.51) (width 0.5) (layer F.Cu) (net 4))
 (segment (start 146.304 -14.12) (end 146.304 -7.62) (width 0.5) (layer F.Cu) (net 2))
 (segment (start 153.924 -9.04) (end 153.924 -2.54) (width 0.5) (layer F.Cu) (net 2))
 (segment (start 169.164 -9.04) (end 169.164 -2.54) (width 0.5) (layer F.Cu) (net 2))
 (segment (start 153.924 -9.04) (end 155.374001 -7.589999) (width 0.5) (layer F.Cu) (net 2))
 (segment (start 155.374001 -7.589999) (end 167.713999 -7.589999) (width 0.5) (layer F.Cu) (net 2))
 (segment (start 167.713999 -7.589999) (end 169.164 -9.04) (width 0.5) (layer F.Cu) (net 2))
 (segment (start 146.304 -7.62) (end 148.723999 -10.039999) (width 0.5) (layer F.Cu) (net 2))
 (segment (start 148.723999 -10.039999) (end 152.924001 -10.039999) (width 0.5) (layer F.Cu) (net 2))
 (segment (start 152.924001 -10.039999) (end 153.924 -9.04) (width 0.5) (layer F.Cu) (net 2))
 (segment (start 138.684 -9.04) (end 141.103999 -6.620001) (width 0.5) (layer F.Cu) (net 2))
 (segment (start 141.103999 -6.620001) (end 145.304001 -6.620001) (width 0.5) (layer F.Cu) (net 2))
 (segment (start 145.304001 -6.620001) (end 146.304 -7.62) (width 0.5) (layer F.Cu) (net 2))
 (segment (start 138.684 -9.04) (end 138.684 -2.54) (width 0.5) (layer F.Cu) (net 2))
 (segment (start 138.684 -13.146002) (end 138.684 -9.04) (width 0.5) (layer F.Cu) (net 2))
 (segment (start 136.260001 -15.570001) (end 138.684 -13.146002) (width 0.5) (layer F.Cu) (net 2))
 (segment (start 87.604 -23.521) (end 90.805 -20.32) (width 0.5) (layer B.Cu) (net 2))
 (via (at 90.805 -20.32) (size 0.8) (drill 0.4) (layers F.Cu B.Cu) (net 2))
 (segment (start 87.604 -24.765) (end 87.604 -23.521) (width 0.5) (layer B.Cu) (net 2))
 (segment (start 95.554999 -15.570001) (end 99.999999 -15.570001) (width 0.5) (layer F.Cu) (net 2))
 (segment (start 90.805 -20.32) (end 95.554999 -15.570001) (width 0.5) (layer F.Cu) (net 2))
 (segment (start 99.999999 -15.570001) (end 136.260001 -15.570001) (width 0.5) (layer F.Cu) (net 2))
 (segment (start 99.338999 -15.570001) (end 99.999999 -15.570001) (width 0.5) (layer F.Cu) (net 2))
 (segment (start 108.204 -9.04) (end 108.204 -2.54) (width 0.5) (layer F.Cu) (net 6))
 (segment (start 110.623999 -6.620001) (end 114.824001 -6.620001) (width 0.5) (layer F.Cu) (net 6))
 (segment (start 108.204 -9.04) (end 110.623999 -6.620001) (width 0.5) (layer F.Cu) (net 6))
 (segment (start 131.064 -7.62) (end 131.064 -14.12) (width 0.5) (layer F.Cu) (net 6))
 (segment (start 123.444 -9.04) (end 125.863999 -6.620001) (width 0.5) (layer F.Cu) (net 6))
 (segment (start 125.863999 -6.620001) (end 130.064001 -6.620001) (width 0.5) (layer F.Cu) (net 6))
 (segment (start 130.064001 -6.620001) (end 131.064 -7.62) (width 0.5) (layer F.Cu) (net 6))
 (segment (start 123.444 -9.04) (end 123.444 -2.54) (width 0.5) (layer F.Cu) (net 6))
 (segment (start 115.824 -14.12) (end 115.824 -7.62) (width 0.5) (layer F.Cu) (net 6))
 (segment (start 115.824 -7.62) (end 118.243999 -10.039999) (width 0.5) (layer F.Cu) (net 6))
 (segment (start 118.243999 -10.039999) (end 122.444001 -10.039999) (width 0.5) (layer F.Cu) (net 6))
 (segment (start 122.444001 -10.039999) (end 123.444 -9.04) (width 0.5) (layer F.Cu) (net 6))
 (segment (start 114.824001 -6.620001) (end 115.824 -7.62) (width 0.5) (layer F.Cu) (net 6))
 (via (at 88.265 -20.32) (size 0.8) (drill 0.4) (layers F.Cu B.Cu) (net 6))
 (segment (start 85.064 -23.521) (end 88.265 -20.32) (width 0.5) (layer B.Cu) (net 6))
 (segment (start 85.064 -24.765) (end 85.064 -23.521) (width 0.5) (layer B.Cu) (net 6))
 (segment (start 99.545 -9.04) (end 100.815 -9.04) (width 0.5) (layer F.Cu) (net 6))
 (segment (start 88.265 -20.32) (end 99.545 -9.04) (width 0.5) (layer F.Cu) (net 6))
 (segment (start 100.815 -9.04) (end 108.204 -9.04) (width 0.5) (layer F.Cu) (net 6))
 (segment (start 100.18 -9.04) (end 100.815 -9.04) (width 0.5) (layer F.Cu) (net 6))
 (segment (start 70.104 -7.62) (end 70.104 -14.12) (width 0.5) (layer F.Cu) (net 7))
 (segment (start 71.554001 -9.070001) (end 77.693999 -9.070001) (width 0.5) (layer F.Cu) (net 7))
 (segment (start 77.693999 -9.070001) (end 77.724 -9.04) (width 0.5) (layer F.Cu) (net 7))
 (segment (start 70.104 -7.62) (end 71.554001 -9.070001) (width 0.5) (layer F.Cu) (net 7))
 (segment (start 84.344001 -6.620001) (end 85.344 -7.62) (width 0.5) (layer F.Cu) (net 7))
 (segment (start 80.143999 -6.620001) (end 84.344001 -6.620001) (width 0.5) (layer F.Cu) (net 7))
 (segment (start 77.724 -9.04) (end 80.143999 -6.620001) (width 0.5) (layer F.Cu) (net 7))
 (segment (start 92.933999 -9.070001) (end 92.964 -9.04) (width 0.5) (layer F.Cu) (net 7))
 (segment (start 86.794001 -9.070001) (end 92.933999 -9.070001) (width 0.5) (layer F.Cu) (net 7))
 (segment (start 85.344 -7.62) (end 86.794001 -9.070001) (width 0.5) (layer F.Cu) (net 7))
 (segment (start 77.724 -9.04) (end 77.724 -2.54) (width 0.5) (layer F.Cu) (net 7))
 (segment (start 85.344 -14.12) (end 85.344 -7.62) (width 0.5) (layer F.Cu) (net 7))
 (segment (start 92.964 -9.04) (end 92.964 -2.54) (width 0.5) (layer F.Cu) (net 7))
 (segment (start 82.524 -16.94) (end 82.752 -16.712) (width 0.5) (layer B.Cu) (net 7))
 (segment (start 82.524 -24.765) (end 82.524 -16.94) (width 0.5) (layer B.Cu) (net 7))
 (segment (start 82.752 -16.712) (end 85.344 -14.12) (width 0.5) (layer B.Cu) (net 7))
 (segment (start 32.004 -9.04) (end 32.004 -2.54) (width 0.5) (layer F.Cu) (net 8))
 (segment (start 39.624 -7.62) (end 39.624 -14.12) (width 0.5) (layer F.Cu) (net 8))
 (segment (start 47.244 -9.04) (end 47.244 -2.54) (width 0.5) (layer F.Cu) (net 8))
 (segment (start 62.484 -9.04) (end 62.484 -2.54) (width 0.5) (layer F.Cu) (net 8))
 (segment (start 39.593999 -7.589999) (end 39.624 -7.62) (width 0.5) (layer F.Cu) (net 8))
 (segment (start 33.454001 -7.589999) (end 39.593999 -7.589999) (width 0.5) (layer F.Cu) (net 8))
 (segment (start 32.004 -9.04) (end 33.454001 -7.589999) (width 0.5) (layer F.Cu) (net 8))
 (segment (start 42.043999 -10.039999) (end 39.624 -7.62) (width 0.5) (layer F.Cu) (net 8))
 (segment (start 46.244001 -10.039999) (end 42.043999 -10.039999) (width 0.5) (layer F.Cu) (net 8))
 (segment (start 47.244 -9.04) (end 46.244001 -10.039999) (width 0.5) (layer F.Cu) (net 8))
 (segment (start 61.033999 -7.589999) (end 62.484 -9.04) (width 0.5) (layer F.Cu) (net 8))
 (segment (start 48.694001 -7.589999) (end 61.033999 -7.589999) (width 0.5) (layer F.Cu) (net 8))
 (segment (start 47.244 -9.04) (end 48.694001 -7.589999) (width 0.5) (layer F.Cu) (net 8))
 (segment (start 76.908999 -23.464999) (end 62.484 -9.04) (width 0.5) (layer F.Cu) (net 8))
 (segment (start 78.683999 -23.464999) (end 76.908999 -23.464999) (width 0.5) (layer F.Cu) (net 8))
 (segment (start 79.984 -24.765) (end 78.683999 -23.464999) (width 0.5) (layer F.Cu) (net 8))
 (segment (start 9.144 -7.62) (end 9.144 -14.12) (width 0.5) (layer F.Cu) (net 9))
 (segment (start 16.764 -2.54) (end 16.764 -9.04) (width 0.5) (layer F.Cu) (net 9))
 (segment (start 24.384 -7.62) (end 24.384 -14.12) (width 0.5) (layer F.Cu) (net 9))
 (segment (start 1.524 -2.54) (end 1.524 -9.04) (width 0.5) (layer F.Cu) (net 9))
 (segment (start 9.113999 -7.589999) (end 9.144 -7.62) (width 0.5) (layer F.Cu) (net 9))
 (segment (start 2.974001 -7.589999) (end 9.113999 -7.589999) (width 0.5) (layer F.Cu) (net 9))
 (segment (start 1.524 -9.04) (end 2.974001 -7.589999) (width 0.5) (layer F.Cu) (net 9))
 (segment (start 16.733999 -9.070001) (end 16.764 -9.04) (width 0.5) (layer F.Cu) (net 9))
 (segment (start 10.594001 -9.070001) (end 16.733999 -9.070001) (width 0.5) (layer F.Cu) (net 9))
 (segment (start 9.144 -7.62) (end 10.594001 -9.070001) (width 0.5) (layer F.Cu) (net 9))
 (segment (start 24.353999 -7.589999) (end 24.384 -7.62) (width 0.5) (layer F.Cu) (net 9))
 (segment (start 18.214001 -7.589999) (end 24.353999 -7.589999) (width 0.5) (layer F.Cu) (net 9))
 (segment (start 16.764 -9.04) (end 18.214001 -7.589999) (width 0.5) (layer F.Cu) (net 9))
 (via (at 64.135 -13.97) (size 0.8) (drill 0.4) (layers F.Cu B.Cu) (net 9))
 (segment (start 74.93 -24.765) (end 64.135 -13.97) (width 0.5) (layer F.Cu) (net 9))
 (segment (start 77.444 -24.765) (end 74.93 -24.765) (width 0.5) (layer F.Cu) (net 9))
 (via (at 50.165 -13.97) (size 0.8) (drill 0.4) (layers F.Cu B.Cu) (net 9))
 (segment (start 64.135 -13.97) (end 50.165 -13.97) (width 0.5) (layer B.Cu) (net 9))
 (segment (start 28.259001 -17.995001) (end 27.992 -17.728) (width 0.5) (layer F.Cu) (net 9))
 (segment (start 46.139999 -17.995001) (end 28.259001 -17.995001) (width 0.5) (layer F.Cu) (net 9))
 (segment (start 50.165 -13.97) (end 46.139999 -17.995001) (width 0.5) (layer F.Cu) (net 9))
 (segment (start 27.992 -17.728) (end 24.384 -14.12) (width 0.5) (layer F.Cu) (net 9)))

